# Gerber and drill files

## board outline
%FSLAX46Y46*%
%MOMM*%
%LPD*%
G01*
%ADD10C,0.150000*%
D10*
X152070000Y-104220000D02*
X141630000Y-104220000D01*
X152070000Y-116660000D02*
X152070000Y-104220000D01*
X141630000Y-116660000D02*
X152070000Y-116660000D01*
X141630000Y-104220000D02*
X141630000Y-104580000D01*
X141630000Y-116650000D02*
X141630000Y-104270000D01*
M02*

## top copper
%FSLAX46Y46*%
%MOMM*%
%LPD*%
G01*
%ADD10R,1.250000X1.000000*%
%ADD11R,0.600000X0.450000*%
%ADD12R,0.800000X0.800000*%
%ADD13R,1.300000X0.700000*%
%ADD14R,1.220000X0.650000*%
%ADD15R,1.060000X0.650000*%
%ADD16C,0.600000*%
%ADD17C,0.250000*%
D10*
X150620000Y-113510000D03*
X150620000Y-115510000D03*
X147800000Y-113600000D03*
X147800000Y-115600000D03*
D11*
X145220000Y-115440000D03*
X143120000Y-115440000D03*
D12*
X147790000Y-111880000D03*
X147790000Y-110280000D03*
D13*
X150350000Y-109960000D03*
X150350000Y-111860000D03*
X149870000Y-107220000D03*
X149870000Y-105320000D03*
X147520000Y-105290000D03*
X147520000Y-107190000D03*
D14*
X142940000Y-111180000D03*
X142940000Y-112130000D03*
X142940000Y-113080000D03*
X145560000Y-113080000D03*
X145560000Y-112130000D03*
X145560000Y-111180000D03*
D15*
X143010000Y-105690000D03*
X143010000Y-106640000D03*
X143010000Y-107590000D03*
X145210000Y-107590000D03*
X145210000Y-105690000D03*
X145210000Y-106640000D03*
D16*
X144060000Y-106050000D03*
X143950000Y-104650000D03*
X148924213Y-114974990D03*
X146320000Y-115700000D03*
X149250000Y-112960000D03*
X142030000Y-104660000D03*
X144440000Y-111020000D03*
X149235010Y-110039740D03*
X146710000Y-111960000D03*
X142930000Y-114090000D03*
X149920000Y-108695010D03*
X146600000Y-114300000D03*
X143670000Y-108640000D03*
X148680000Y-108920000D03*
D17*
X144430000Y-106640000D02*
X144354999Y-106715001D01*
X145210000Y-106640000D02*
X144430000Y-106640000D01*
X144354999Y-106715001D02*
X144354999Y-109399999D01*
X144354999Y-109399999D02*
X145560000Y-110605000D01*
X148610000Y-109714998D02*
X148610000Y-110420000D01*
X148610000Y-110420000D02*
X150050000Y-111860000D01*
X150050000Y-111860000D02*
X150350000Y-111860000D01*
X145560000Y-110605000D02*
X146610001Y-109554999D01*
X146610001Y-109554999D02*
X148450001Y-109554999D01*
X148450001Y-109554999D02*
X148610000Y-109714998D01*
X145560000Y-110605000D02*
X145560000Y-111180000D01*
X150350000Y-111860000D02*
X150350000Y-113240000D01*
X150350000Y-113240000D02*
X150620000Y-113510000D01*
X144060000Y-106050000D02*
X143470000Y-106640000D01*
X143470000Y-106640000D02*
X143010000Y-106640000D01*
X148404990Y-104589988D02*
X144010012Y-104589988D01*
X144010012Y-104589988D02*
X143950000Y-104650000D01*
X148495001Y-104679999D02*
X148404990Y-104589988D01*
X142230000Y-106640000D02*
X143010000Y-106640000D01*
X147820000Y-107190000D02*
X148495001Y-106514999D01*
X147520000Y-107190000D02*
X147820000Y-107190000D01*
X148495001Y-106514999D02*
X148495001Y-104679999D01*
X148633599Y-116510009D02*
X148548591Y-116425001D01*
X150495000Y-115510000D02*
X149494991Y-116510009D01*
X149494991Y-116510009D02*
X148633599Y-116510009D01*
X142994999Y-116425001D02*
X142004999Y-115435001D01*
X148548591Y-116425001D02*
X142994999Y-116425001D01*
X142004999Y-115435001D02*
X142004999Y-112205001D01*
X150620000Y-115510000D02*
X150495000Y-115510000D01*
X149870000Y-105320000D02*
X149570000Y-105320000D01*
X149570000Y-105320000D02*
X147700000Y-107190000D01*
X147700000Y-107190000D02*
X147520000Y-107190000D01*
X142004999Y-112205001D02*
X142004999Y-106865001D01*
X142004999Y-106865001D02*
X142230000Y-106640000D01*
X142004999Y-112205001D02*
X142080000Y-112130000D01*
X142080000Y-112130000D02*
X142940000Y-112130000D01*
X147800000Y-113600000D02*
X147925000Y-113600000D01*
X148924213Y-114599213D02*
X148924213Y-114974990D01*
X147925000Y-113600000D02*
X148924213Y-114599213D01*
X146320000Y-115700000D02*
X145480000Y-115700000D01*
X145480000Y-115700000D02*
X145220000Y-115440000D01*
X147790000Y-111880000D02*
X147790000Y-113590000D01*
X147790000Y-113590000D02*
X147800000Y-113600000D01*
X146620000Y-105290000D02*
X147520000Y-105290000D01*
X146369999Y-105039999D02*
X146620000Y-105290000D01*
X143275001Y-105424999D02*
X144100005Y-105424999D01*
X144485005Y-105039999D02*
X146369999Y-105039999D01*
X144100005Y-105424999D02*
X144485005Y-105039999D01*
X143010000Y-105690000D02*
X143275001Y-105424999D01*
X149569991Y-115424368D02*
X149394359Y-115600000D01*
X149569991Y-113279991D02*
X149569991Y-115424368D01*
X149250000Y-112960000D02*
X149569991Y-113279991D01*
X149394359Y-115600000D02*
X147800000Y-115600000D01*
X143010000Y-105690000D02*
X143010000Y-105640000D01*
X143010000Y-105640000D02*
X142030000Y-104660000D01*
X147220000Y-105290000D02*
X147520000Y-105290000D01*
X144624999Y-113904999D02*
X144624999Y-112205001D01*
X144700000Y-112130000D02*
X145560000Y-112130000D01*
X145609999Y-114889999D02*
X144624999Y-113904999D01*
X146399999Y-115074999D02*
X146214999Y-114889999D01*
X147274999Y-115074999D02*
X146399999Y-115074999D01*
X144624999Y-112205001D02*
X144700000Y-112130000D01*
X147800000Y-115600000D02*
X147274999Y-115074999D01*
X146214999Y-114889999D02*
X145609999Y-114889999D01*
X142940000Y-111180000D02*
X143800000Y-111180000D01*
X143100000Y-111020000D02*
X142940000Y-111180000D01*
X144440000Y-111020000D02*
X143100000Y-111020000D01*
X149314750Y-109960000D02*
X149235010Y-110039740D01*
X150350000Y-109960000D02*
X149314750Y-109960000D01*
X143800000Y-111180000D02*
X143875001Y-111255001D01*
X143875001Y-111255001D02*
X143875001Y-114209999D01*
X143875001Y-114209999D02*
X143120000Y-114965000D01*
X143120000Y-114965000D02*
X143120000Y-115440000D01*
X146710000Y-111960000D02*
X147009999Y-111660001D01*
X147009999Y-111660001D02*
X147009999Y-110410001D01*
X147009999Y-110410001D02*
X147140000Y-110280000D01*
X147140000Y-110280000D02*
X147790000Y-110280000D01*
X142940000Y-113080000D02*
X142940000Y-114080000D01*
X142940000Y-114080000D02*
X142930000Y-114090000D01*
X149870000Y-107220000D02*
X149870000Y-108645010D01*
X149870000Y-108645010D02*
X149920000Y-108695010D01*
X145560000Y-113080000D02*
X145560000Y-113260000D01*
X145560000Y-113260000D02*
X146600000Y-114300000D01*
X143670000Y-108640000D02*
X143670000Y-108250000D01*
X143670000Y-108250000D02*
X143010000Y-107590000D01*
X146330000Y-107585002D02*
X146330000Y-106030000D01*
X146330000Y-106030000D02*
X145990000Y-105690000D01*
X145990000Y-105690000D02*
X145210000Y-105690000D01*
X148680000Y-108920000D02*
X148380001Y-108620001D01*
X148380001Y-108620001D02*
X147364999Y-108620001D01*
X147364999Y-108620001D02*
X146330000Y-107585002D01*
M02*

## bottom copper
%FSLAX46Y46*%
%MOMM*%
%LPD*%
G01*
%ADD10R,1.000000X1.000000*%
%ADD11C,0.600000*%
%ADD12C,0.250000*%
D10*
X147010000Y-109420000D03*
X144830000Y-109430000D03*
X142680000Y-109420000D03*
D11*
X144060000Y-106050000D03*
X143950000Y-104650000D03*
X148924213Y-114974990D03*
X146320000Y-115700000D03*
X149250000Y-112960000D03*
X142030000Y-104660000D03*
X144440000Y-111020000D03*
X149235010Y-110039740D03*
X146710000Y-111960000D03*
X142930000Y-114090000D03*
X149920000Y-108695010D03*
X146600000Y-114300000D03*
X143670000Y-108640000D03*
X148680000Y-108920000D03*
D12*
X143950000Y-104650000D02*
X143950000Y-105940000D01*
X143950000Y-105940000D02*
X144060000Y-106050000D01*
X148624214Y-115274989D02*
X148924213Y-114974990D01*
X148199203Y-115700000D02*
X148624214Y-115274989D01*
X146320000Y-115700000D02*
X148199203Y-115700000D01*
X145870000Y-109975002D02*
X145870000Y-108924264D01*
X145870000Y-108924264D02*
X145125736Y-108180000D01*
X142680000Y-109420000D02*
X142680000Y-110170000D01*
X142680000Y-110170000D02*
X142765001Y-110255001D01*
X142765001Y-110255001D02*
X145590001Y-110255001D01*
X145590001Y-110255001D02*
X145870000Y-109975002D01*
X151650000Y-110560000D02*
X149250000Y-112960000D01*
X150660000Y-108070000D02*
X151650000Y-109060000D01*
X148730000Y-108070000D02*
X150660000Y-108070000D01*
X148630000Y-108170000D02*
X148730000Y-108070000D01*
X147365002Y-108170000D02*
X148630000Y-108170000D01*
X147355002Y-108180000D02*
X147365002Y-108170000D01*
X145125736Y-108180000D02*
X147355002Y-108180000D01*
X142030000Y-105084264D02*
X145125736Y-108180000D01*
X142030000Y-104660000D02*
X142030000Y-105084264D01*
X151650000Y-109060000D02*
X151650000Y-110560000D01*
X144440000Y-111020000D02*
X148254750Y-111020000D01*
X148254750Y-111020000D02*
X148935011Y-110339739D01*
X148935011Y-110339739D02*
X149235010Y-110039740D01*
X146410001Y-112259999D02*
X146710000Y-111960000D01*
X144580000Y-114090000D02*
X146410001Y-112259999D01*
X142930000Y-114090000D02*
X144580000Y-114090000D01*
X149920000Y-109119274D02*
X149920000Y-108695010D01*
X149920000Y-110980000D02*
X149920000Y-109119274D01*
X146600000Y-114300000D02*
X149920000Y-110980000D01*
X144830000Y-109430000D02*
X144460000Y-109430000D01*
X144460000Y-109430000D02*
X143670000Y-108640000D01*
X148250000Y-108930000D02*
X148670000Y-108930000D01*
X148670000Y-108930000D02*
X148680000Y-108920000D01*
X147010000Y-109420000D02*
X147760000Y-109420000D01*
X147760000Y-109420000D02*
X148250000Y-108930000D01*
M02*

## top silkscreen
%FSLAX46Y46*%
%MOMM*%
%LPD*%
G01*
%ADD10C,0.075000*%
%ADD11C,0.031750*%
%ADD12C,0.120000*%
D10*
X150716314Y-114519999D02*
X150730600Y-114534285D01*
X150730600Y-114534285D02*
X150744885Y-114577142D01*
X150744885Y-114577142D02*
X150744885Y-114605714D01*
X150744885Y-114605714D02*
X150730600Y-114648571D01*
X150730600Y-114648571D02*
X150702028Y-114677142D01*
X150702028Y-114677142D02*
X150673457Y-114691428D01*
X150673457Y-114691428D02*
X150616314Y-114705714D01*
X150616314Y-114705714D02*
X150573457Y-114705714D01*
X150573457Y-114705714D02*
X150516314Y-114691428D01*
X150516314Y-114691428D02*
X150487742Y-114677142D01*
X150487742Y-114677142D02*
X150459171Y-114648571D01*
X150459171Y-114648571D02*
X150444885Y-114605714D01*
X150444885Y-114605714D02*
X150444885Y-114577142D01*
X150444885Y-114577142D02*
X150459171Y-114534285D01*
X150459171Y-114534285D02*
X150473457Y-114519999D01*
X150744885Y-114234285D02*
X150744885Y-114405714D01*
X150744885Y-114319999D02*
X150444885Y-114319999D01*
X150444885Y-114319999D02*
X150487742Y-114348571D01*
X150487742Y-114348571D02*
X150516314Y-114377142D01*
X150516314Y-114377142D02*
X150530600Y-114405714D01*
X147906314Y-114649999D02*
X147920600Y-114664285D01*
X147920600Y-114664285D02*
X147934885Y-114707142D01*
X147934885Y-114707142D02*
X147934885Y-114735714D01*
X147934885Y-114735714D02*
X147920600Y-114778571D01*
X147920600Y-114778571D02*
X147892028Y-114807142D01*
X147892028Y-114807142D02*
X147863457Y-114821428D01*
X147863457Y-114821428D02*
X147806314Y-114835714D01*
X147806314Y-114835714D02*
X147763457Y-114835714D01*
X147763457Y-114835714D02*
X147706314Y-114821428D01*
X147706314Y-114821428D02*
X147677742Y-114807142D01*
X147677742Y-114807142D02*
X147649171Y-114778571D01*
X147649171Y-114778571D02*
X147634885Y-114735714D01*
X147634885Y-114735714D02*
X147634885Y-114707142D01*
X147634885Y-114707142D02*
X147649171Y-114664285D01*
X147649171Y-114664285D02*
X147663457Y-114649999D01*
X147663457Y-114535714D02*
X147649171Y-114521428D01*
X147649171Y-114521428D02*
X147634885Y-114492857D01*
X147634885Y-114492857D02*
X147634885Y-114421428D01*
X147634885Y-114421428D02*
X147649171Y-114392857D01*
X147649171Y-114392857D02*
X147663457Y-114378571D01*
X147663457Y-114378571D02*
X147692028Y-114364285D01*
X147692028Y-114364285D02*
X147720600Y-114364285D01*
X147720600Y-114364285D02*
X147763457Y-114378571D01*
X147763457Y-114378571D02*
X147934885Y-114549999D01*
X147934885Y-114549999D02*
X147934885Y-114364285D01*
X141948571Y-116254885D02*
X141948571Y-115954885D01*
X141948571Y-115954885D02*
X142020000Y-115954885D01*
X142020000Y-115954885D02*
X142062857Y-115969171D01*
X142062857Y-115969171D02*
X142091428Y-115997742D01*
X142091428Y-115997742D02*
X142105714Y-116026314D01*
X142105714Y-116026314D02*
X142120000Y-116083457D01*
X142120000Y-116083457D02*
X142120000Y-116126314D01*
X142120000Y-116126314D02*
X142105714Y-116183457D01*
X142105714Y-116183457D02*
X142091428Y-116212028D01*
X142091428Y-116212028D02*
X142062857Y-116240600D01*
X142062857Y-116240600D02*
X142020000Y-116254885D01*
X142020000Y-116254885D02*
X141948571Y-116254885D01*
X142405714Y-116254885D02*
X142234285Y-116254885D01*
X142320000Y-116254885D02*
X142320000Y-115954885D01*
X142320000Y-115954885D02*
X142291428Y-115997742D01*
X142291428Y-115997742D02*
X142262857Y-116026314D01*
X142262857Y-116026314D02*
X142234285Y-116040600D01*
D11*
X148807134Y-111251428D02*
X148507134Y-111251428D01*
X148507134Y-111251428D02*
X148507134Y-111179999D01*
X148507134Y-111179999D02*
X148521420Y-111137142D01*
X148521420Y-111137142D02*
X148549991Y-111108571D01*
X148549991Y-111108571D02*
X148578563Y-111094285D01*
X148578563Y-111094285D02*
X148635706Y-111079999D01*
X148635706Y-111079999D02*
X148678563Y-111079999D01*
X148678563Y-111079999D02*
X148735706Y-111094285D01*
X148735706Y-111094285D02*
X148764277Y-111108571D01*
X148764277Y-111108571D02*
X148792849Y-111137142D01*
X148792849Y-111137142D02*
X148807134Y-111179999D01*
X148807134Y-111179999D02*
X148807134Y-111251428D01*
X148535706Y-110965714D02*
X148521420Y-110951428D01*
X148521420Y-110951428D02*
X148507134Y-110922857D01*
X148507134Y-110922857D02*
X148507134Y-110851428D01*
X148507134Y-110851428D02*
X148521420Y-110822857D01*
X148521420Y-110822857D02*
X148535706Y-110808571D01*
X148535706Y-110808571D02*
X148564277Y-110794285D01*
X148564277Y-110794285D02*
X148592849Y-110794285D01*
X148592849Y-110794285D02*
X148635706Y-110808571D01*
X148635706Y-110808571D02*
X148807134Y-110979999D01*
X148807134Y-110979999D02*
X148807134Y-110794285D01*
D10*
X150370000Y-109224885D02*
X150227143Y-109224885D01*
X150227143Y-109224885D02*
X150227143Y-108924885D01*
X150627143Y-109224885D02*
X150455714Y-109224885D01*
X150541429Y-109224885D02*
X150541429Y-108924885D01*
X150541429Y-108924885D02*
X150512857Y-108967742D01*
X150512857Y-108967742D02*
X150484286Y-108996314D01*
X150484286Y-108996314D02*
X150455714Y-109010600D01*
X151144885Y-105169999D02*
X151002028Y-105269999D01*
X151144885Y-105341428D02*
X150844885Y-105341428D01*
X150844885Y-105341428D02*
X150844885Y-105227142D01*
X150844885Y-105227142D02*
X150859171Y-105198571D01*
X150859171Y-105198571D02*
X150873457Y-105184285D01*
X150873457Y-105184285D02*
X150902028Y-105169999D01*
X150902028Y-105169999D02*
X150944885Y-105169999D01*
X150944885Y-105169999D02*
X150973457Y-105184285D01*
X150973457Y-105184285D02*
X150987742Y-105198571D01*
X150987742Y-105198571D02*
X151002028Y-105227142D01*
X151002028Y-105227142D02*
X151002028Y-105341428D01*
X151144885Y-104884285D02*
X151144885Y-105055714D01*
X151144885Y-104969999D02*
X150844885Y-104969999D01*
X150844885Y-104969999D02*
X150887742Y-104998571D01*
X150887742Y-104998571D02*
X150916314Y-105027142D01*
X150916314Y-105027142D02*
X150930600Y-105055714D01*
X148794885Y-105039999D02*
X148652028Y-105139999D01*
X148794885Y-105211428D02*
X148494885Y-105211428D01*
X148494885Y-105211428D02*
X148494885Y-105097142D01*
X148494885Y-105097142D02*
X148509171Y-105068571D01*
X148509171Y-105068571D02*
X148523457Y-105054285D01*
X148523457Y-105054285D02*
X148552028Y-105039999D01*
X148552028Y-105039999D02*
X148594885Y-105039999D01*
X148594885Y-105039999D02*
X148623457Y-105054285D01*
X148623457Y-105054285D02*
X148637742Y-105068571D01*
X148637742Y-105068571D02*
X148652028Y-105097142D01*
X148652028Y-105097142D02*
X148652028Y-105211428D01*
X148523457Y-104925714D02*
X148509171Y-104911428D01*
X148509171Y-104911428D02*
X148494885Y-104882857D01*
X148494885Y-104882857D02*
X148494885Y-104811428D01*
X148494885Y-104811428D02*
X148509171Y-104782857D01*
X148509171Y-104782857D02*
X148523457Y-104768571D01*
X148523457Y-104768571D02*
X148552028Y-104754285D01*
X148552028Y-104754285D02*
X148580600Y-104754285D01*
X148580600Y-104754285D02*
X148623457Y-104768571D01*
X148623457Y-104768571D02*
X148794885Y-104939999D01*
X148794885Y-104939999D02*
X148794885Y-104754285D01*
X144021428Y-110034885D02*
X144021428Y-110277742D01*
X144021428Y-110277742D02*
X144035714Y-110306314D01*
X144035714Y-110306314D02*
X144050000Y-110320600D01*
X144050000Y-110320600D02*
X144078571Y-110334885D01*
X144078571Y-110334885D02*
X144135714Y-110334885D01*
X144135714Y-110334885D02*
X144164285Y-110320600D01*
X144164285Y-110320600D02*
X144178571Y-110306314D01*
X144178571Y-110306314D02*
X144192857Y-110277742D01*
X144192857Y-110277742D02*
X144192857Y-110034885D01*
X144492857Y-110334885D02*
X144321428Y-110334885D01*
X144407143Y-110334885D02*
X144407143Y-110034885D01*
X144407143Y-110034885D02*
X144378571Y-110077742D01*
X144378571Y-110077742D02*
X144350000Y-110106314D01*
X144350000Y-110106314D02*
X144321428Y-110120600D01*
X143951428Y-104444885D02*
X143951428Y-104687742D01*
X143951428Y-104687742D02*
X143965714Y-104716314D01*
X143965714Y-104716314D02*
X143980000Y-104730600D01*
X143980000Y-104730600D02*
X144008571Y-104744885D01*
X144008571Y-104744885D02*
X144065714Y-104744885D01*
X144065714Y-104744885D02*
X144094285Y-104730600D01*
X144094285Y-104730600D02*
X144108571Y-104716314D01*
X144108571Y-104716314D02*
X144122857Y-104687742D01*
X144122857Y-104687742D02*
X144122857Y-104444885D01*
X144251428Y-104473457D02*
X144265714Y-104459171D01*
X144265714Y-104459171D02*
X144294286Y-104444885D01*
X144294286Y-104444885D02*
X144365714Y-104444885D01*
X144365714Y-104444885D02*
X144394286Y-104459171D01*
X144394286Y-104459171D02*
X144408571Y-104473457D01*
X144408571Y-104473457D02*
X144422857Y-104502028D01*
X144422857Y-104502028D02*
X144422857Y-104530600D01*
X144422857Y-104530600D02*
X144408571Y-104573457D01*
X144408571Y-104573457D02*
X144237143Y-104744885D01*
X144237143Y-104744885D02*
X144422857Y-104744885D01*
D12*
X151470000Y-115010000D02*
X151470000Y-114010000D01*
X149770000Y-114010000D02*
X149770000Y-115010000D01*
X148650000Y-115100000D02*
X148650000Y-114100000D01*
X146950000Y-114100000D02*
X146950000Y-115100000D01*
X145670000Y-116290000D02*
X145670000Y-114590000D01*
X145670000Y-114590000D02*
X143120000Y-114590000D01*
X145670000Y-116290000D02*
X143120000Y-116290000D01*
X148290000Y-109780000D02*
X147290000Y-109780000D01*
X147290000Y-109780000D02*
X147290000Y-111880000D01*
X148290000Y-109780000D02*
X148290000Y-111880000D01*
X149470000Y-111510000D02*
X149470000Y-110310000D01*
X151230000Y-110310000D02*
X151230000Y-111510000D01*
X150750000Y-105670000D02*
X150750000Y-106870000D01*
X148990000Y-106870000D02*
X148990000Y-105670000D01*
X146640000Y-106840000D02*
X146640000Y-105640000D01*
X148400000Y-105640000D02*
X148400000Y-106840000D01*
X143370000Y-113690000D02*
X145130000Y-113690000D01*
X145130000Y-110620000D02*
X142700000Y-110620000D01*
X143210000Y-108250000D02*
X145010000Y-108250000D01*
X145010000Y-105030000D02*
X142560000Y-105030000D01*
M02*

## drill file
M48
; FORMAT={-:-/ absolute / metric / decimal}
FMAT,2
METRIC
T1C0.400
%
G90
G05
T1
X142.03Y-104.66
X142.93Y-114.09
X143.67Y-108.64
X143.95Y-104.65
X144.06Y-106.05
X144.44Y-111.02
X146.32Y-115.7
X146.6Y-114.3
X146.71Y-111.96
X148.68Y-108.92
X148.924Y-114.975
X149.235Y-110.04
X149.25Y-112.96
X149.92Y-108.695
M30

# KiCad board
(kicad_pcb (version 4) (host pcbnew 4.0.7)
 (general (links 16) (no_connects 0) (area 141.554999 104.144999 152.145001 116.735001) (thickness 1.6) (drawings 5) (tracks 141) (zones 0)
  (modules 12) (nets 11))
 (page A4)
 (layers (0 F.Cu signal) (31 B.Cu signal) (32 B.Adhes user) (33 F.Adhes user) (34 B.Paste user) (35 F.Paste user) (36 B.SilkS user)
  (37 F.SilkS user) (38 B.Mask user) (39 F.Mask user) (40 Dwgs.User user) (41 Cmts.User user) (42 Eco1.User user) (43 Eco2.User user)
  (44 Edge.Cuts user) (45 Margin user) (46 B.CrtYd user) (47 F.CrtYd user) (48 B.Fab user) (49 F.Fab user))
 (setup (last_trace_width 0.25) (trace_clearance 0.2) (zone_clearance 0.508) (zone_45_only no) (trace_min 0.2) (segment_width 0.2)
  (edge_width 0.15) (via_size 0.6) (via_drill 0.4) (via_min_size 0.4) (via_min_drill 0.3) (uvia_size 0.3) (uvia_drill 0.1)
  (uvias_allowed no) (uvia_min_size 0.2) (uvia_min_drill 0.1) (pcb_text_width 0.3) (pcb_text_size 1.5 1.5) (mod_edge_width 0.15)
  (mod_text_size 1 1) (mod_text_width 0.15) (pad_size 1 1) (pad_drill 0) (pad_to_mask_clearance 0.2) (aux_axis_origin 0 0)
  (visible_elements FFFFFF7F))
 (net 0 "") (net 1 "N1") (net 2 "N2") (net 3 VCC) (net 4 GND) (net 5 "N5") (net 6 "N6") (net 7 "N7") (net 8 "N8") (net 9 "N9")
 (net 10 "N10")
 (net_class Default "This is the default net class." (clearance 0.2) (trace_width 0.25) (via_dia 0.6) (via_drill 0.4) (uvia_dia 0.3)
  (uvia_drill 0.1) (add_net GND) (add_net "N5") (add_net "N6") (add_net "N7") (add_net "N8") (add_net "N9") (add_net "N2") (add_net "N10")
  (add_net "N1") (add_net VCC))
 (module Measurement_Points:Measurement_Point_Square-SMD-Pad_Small (layer B.Cu) (at 147.01 109.42)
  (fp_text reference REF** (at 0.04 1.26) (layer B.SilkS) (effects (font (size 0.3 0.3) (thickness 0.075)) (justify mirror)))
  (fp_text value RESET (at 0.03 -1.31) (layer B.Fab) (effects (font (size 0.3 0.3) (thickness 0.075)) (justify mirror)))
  (pad 1 smd rect (at 0 0) (size 1 1) (layers B.Cu B.Mask) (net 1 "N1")))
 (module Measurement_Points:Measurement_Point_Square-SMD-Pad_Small (layer B.Cu) (at 144.83 109.43)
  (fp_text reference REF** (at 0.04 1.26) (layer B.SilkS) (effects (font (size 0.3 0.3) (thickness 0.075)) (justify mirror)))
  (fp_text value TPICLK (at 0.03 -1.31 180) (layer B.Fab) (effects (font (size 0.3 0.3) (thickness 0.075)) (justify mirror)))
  (pad 1 smd rect (at 0 0) (size 1 1) (layers B.Cu B.Mask) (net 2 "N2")))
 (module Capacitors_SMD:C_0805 (layer F.Cu) (at 150.62 114.51 270)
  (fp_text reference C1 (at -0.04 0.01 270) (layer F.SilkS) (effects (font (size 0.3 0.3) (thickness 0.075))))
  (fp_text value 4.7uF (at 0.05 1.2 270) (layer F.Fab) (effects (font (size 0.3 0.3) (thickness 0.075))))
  (fp_line (start 0.5 -0.85) (end -0.5 -0.85) (layer F.SilkS) (width 0.12))
  (fp_line (start -0.5 0.85) (end 0.5 0.85) (layer F.SilkS) (width 0.12))
  (pad 1 smd rect (at -1 0 270) (size 1 1.25) (layers F.Cu F.Paste F.Mask) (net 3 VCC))
  (pad 2 smd rect (at 1 0 270) (size 1 1.25) (layers F.Cu F.Paste F.Mask) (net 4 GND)))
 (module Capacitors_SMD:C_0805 (layer F.Cu) (at 147.8 114.6 270)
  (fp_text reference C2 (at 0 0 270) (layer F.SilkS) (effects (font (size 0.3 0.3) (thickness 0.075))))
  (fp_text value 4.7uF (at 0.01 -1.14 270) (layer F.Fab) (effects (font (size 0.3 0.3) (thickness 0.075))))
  (fp_line (start 0.5 -0.85) (end -0.5 -0.85) (layer F.SilkS) (width 0.12))
  (fp_line (start -0.5 0.85) (end 0.5 0.85) (layer F.SilkS) (width 0.12))
  (pad 1 smd rect (at -1 0 270) (size 1 1.25) (layers F.Cu F.Paste F.Mask) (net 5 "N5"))
  (pad 2 smd rect (at 1 0 270) (size 1 1.25) (layers F.Cu F.Paste F.Mask) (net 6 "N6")))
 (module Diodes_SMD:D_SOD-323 (layer F.Cu) (at 144.17 115.44 180)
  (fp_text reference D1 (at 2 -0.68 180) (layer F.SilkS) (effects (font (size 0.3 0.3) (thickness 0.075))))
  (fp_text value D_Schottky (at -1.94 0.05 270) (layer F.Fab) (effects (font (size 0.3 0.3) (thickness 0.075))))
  (fp_line (start -1.5 -0.85) (end -1.5 0.85) (layer F.SilkS) (width 0.12))
  (fp_line (start -1.5 0.85) (end 1.05 0.85) (layer F.SilkS) (width 0.12))
  (fp_line (start -1.5 -0.85) (end 1.05 -0.85) (layer F.SilkS) (width 0.12))
  (pad 1 smd rect (at -1.05 0 180) (size 0.6 0.45) (layers F.Cu F.Paste F.Mask) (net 5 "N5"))
  (pad 2 smd rect (at 1.05 0 180) (size 0.6 0.45) (layers F.Cu F.Paste F.Mask) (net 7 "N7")))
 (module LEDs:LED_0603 (layer F.Cu) (at 147.79 111.08 270)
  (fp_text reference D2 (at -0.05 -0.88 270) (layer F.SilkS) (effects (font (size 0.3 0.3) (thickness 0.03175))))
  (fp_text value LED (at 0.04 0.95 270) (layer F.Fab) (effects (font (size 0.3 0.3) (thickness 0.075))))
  (fp_line (start -1.3 -0.5) (end -1.3 0.5) (layer F.SilkS) (width 0.12))
  (fp_line (start -1.3 0.5) (end 0.8 0.5) (layer F.SilkS) (width 0.12))
  (fp_line (start -1.3 -0.5) (end 0.8 -0.5) (layer F.SilkS) (width 0.12))
  (pad 2 smd rect (at 0.8 0 90) (size 0.8 0.8) (layers F.Cu F.Paste F.Mask) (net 5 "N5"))
  (pad 1 smd rect (at -0.8 0 90) (size 0.8 0.8) (layers F.Cu F.Paste F.Mask) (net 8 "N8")))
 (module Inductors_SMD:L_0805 (layer F.Cu) (at 150.35 110.91 270)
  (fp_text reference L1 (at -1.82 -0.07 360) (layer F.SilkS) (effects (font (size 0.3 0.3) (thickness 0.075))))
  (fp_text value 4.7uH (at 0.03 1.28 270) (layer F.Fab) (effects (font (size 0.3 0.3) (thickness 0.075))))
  (fp_line (start 0.6 0.88) (end -0.6 0.88) (layer F.SilkS) (width 0.12))
  (fp_line (start -0.6 -0.88) (end 0.6 -0.88) (layer F.SilkS) (width 0.12))
  (pad 1 smd rect (at -0.95 0 270) (size 0.7 1.3) (layers F.Cu F.Paste F.Mask) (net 7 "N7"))
  (pad 2 smd rect (at 0.95 0 270) (size 0.7 1.3) (layers F.Cu F.Paste F.Mask) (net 3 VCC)))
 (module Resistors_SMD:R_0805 (layer F.Cu) (at 149.87 106.27 90)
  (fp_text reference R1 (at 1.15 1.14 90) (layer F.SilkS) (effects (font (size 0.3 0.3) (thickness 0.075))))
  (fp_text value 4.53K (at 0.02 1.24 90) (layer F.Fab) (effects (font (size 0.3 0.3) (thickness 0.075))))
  (fp_line (start 0.6 0.88) (end -0.6 0.88) (layer F.SilkS) (width 0.12))
  (fp_line (start -0.6 -0.88) (end 0.6 -0.88) (layer F.SilkS) (width 0.12))
  (pad 1 smd rect (at -0.95 0 90) (size 0.7 1.3) (layers F.Cu F.Paste F.Mask) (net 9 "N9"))
  (pad 2 smd rect (at 0.95 0 90) (size 0.7 1.3) (layers F.Cu F.Paste F.Mask) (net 4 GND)))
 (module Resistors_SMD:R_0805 (layer F.Cu) (at 147.52 106.24 270)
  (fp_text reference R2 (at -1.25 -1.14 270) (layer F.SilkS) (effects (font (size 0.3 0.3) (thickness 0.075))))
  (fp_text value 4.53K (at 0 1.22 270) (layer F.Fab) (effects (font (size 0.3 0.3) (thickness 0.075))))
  (fp_line (start 0.6 0.88) (end -0.6 0.88) (layer F.SilkS) (width 0.12))
  (fp_line (start -0.6 -0.88) (end 0.6 -0.88) (layer F.SilkS) (width 0.12))
  (pad 1 smd rect (at -0.95 0 270) (size 0.7 1.3) (layers F.Cu F.Paste F.Mask) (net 6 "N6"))
  (pad 2 smd rect (at 0.95 0 270) (size 0.7 1.3) (layers F.Cu F.Paste F.Mask) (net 4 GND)))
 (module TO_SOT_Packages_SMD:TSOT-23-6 (layer F.Cu) (at 144.25 112.13)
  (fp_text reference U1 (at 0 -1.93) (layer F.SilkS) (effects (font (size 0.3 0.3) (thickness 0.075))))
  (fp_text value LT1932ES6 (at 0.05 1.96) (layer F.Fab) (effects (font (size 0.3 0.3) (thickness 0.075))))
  (fp_line (start -0.88 1.56) (end 0.88 1.56) (layer F.SilkS) (width 0.12))
  (fp_line (start 0.88 -1.51) (end -1.55 -1.51) (layer F.SilkS) (width 0.12))
  (pad 1 smd rect (at -1.31 -0.95) (size 1.22 0.65) (layers F.Cu F.Paste F.Mask) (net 7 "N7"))
  (pad 2 smd rect (at -1.31 0) (size 1.22 0.65) (layers F.Cu F.Paste F.Mask) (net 4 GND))
  (pad 3 smd rect (at -1.31 0.95) (size 1.22 0.65) (layers F.Cu F.Paste F.Mask) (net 8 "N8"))
  (pad 4 smd rect (at 1.31 0.95) (size 1.22 0.65) (layers F.Cu F.Paste F.Mask) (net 9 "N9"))
  (pad 5 smd rect (at 1.31 0) (size 1.22 0.65) (layers F.Cu F.Paste F.Mask) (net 6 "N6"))
  (pad 6 smd rect (at 1.31 -0.95) (size 1.22 0.65) (layers F.Cu F.Paste F.Mask) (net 3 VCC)))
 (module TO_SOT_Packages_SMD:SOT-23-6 (layer F.Cu) (at 144.11 106.64)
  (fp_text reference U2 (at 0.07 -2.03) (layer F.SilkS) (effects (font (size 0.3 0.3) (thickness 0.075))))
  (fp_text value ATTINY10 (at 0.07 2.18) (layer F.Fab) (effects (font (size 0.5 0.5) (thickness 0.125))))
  (fp_line (start -0.9 1.61) (end 0.9 1.61) (layer F.SilkS) (width 0.12))
  (fp_line (start 0.9 -1.61) (end -1.55 -1.61) (layer F.SilkS) (width 0.12))
  (pad 1 smd rect (at -1.1 -0.95) (size 1.06 0.65) (layers F.Cu F.Paste F.Mask) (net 6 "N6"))
  (pad 2 smd rect (at -1.1 0) (size 1.06 0.65) (layers F.Cu F.Paste F.Mask) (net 4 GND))
  (pad 3 smd rect (at -1.1 0.95) (size 1.06 0.65) (layers F.Cu F.Paste F.Mask) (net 2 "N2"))
  (pad 4 smd rect (at 1.1 0.95) (size 1.06 0.65) (layers F.Cu F.Paste F.Mask) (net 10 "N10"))
  (pad 6 smd rect (at 1.1 -0.95) (size 1.06 0.65) (layers F.Cu F.Paste F.Mask) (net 1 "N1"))
  (pad 5 smd rect (at 1.1 0) (size 1.06 0.65) (layers F.Cu F.Paste F.Mask) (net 3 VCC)))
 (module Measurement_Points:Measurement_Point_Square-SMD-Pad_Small (layer B.Cu) (at 142.68 109.42)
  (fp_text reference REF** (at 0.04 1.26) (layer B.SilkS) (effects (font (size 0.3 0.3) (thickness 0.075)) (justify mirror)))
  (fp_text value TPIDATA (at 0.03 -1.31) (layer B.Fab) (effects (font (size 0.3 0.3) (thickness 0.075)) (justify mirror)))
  (pad 1 smd rect (at 0 0) (size 1 1) (layers B.Cu B.Mask) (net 6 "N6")))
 (gr_line (start 152.07 104.22) (end 141.63 104.22) (angle 90) (layer Edge.Cuts) (width 0.15))
 (gr_line (start 152.07 116.66) (end 152.07 104.22) (angle 90) (layer Edge.Cuts) (width 0.15))
 (gr_line (start 141.63 116.66) (end 152.07 116.66) (angle 90) (layer Edge.Cuts) (width 0.15))
 (gr_line (start 141.63 104.22) (end 141.63 104.58) (angle 90) (layer Edge.Cuts) (width 0.15))
 (gr_line (start 141.63 116.65) (end 141.63 104.27) (angle 90) (layer Edge.Cuts) (width 0.15))
 (segment (start 144.43 106.64) (end 144.354999 106.715001) (width 0.25) (layer F.Cu) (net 3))
 (segment (start 145.21 106.64) (end 144.43 106.64) (width 0.25) (layer F.Cu) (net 3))
 (segment (start 144.354999 106.715001) (end 144.354999 109.399999) (width 0.25) (layer F.Cu) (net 3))
 (segment (start 144.354999 109.399999) (end 145.56 110.605) (width 0.25) (layer F.Cu) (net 3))
 (segment (start 148.61 109.714998) (end 148.61 110.42) (width 0.25) (layer F.Cu) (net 3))
 (segment (start 148.61 110.42) (end 150.05 111.86) (width 0.25) (layer F.Cu) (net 3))
 (segment (start 150.05 111.86) (end 150.35 111.86) (width 0.25) (layer F.Cu) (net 3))
 (segment (start 145.56 110.605) (end 146.610001 109.554999) (width 0.25) (layer F.Cu) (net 3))
 (segment (start 146.610001 109.554999) (end 148.450001 109.554999) (width 0.25) (layer F.Cu) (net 3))
 (segment (start 148.450001 109.554999) (end 148.61 109.714998) (width 0.25) (layer F.Cu) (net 3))
 (segment (start 145.56 110.605) (end 145.56 111.18) (width 0.25) (layer F.Cu) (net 3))
 (segment (start 150.35 111.86) (end 150.35 113.24) (width 0.25) (layer F.Cu) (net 3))
 (segment (start 150.35 113.24) (end 150.62 113.51) (width 0.25) (layer F.Cu) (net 3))
 (segment (start 144.06 106.05) (end 143.47 106.64) (width 0.25) (layer F.Cu) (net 4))
 (segment (start 143.47 106.64) (end 143.01 106.64) (width 0.25) (layer F.Cu) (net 4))
 (segment (start 143.95 104.65) (end 143.95 105.94) (width 0.25) (layer B.Cu) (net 4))
 (segment (start 143.95 105.94) (end 144.06 106.05) (width 0.25) (layer B.Cu) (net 4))
 (via (at 144.06 106.05) (size 0.6) (drill 0.4) (layers F.Cu B.Cu) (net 4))
 (segment (start 148.40499 104.589988) (end 144.010012 104.589988) (width 0.25) (layer F.Cu) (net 4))
 (segment (start 144.010012 104.589988) (end 143.95 104.65) (width 0.25) (layer F.Cu) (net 4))
 (segment (start 148.495001 104.679999) (end 148.40499 104.589988) (width 0.25) (layer F.Cu) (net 4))
 (via (at 143.95 104.65) (size 0.6) (drill 0.4) (layers F.Cu B.Cu) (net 4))
 (segment (start 142.23 106.64) (end 143.01 106.64) (width 0.25) (layer F.Cu) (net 4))
 (segment (start 147.82 107.19) (end 148.495001 106.514999) (width 0.25) (layer F.Cu) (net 4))
 (segment (start 147.52 107.19) (end 147.82 107.19) (width 0.25) (layer F.Cu) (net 4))
 (segment (start 148.495001 106.514999) (end 148.495001 104.679999) (width 0.25) (layer F.Cu) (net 4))
 (segment (start 148.633599 116.510009) (end 148.548591 116.425001) (width 0.25) (layer F.Cu) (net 4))
 (segment (start 150.495 115.51) (end 149.494991 116.510009) (width 0.25) (layer F.Cu) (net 4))
 (segment (start 149.494991 116.510009) (end 148.633599 116.510009) (width 0.25) (layer F.Cu) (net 4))
 (segment (start 142.994999 116.425001) (end 142.004999 115.435001) (width 0.25) (layer F.Cu) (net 4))
 (segment (start 148.548591 116.425001) (end 142.994999 116.425001) (width 0.25) (layer F.Cu) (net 4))
 (segment (start 142.004999 115.435001) (end 142.004999 112.205001) (width 0.25) (layer F.Cu) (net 4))
 (segment (start 150.62 115.51) (end 150.495 115.51) (width 0.25) (layer F.Cu) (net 4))
 (segment (start 149.87 105.32) (end 149.57 105.32) (width 0.25) (layer F.Cu) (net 4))
 (segment (start 149.57 105.32) (end 147.7 107.19) (width 0.25) (layer F.Cu) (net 4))
 (segment (start 147.7 107.19) (end 147.52 107.19) (width 0.25) (layer F.Cu) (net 4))
 (segment (start 142.004999 112.205001) (end 142.004999 106.865001) (width 0.25) (layer F.Cu) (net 4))
 (segment (start 142.004999 106.865001) (end 142.23 106.64) (width 0.25) (layer F.Cu) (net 4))
 (segment (start 142.004999 112.205001) (end 142.08 112.13) (width 0.25) (layer F.Cu) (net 4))
 (segment (start 142.08 112.13) (end 142.94 112.13) (width 0.25) (layer F.Cu) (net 4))
 (segment (start 148.624214 115.274989) (end 148.924213 114.97499) (width 0.25) (layer B.Cu) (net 5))
 (segment (start 148.199203 115.7) (end 148.624214 115.274989) (width 0.25) (layer B.Cu) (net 5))
 (segment (start 147.8 113.6) (end 147.925 113.6) (width 0.25) (layer F.Cu) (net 5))
 (segment (start 146.32 115.7) (end 148.199203 115.7) (width 0.25) (layer B.Cu) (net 5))
 (segment (start 148.924213 114.599213) (end 148.924213 114.97499) (width 0.25) (layer F.Cu) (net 5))
 (segment (start 147.925 113.6) (end 148.924213 114.599213) (width 0.25) (layer F.Cu) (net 5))
 (via (at 148.924213 114.97499) (size 0.6) (drill 0.4) (layers F.Cu B.Cu) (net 5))
 (segment (start 146.32 115.7) (end 145.48 115.7) (width 0.25) (layer F.Cu) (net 5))
 (segment (start 145.48 115.7) (end 145.22 115.44) (width 0.25) (layer F.Cu) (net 5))
 (via (at 146.32 115.7) (size 0.6) (drill 0.4) (layers F.Cu B.Cu) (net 5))
 (segment (start 147.79 111.88) (end 147.79 113.59) (width 0.25) (layer F.Cu) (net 5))
 (segment (start 147.79 113.59) (end 147.8 113.6) (width 0.25) (layer F.Cu) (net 5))
 (segment (start 145.87 109.975002) (end 145.87 108.924264) (width 0.25) (layer B.Cu) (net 6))
 (segment (start 145.87 108.924264) (end 145.125736 108.18) (width 0.25) (layer B.Cu) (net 6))
 (segment (start 142.68 109.42) (end 142.68 110.17) (width 0.25) (layer B.Cu) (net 6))
 (segment (start 142.68 110.17) (end 142.765001 110.255001) (width 0.25) (layer B.Cu) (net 6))
 (segment (start 142.765001 110.255001) (end 145.590001 110.255001) (width 0.25) (layer B.Cu) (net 6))
 (segment (start 145.590001 110.255001) (end 145.87 109.975002) (width 0.25) (layer B.Cu) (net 6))
 (segment (start 146.62 105.29) (end 147.52 105.29) (width 0.25) (layer F.Cu) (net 6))
 (segment (start 146.369999 105.039999) (end 146.62 105.29) (width 0.25) (layer F.Cu) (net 6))
 (segment (start 143.275001 105.424999) (end 144.100005 105.424999) (width 0.25) (layer F.Cu) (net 6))
 (segment (start 144.485005 105.039999) (end 146.369999 105.039999) (width 0.25) (layer F.Cu) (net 6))
 (segment (start 144.100005 105.424999) (end 144.485005 105.039999) (width 0.25) (layer F.Cu) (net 6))
 (segment (start 143.01 105.69) (end 143.275001 105.424999) (width 0.25) (layer F.Cu) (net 6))
 (segment (start 151.65 110.56) (end 149.25 112.96) (width 0.25) (layer B.Cu) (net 6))
 (segment (start 150.66 108.07) (end 151.65 109.06) (width 0.25) (layer B.Cu) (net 6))
 (segment (start 148.73 108.07) (end 150.66 108.07) (width 0.25) (layer B.Cu) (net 6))
 (segment (start 148.63 108.17) (end 148.73 108.07) (width 0.25) (layer B.Cu) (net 6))
 (segment (start 147.365002 108.17) (end 148.63 108.17) (width 0.25) (layer B.Cu) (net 6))
 (segment (start 147.355002 108.18) (end 147.365002 108.17) (width 0.25) (layer B.Cu) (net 6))
 (segment (start 145.125736 108.18) (end 147.355002 108.18) (width 0.25) (layer B.Cu) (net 6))
 (segment (start 142.03 105.084264) (end 145.125736 108.18) (width 0.25) (layer B.Cu) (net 6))
 (segment (start 142.03 104.66) (end 142.03 105.084264) (width 0.25) (layer B.Cu) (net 6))
 (segment (start 151.65 109.06) (end 151.65 110.56) (width 0.25) (layer B.Cu) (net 6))
 (segment (start 149.569991 115.424368) (end 149.394359 115.6) (width 0.25) (layer F.Cu) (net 6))
 (segment (start 149.569991 113.279991) (end 149.569991 115.424368) (width 0.25) (layer F.Cu) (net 6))
 (segment (start 149.25 112.96) (end 149.569991 113.279991) (width 0.25) (layer F.Cu) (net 6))
 (segment (start 149.394359 115.6) (end 147.8 115.6) (width 0.25) (layer F.Cu) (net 6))
 (via (at 149.25 112.96) (size 0.6) (drill 0.4) (layers F.Cu B.Cu) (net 6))
 (segment (start 143.01 105.69) (end 143.01 105.64) (width 0.25) (layer F.Cu) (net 6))
 (via (at 142.03 104.66) (size 0.6) (drill 0.4) (layers F.Cu B.Cu) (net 6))
 (segment (start 143.01 105.64) (end 142.03 104.66) (width 0.25) (layer F.Cu) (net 6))
 (segment (start 147.22 105.29) (end 147.52 105.29) (width 0.25) (layer F.Cu) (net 6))
 (segment (start 144.624999 113.904999) (end 144.624999 112.205001) (width 0.25) (layer F.Cu) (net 6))
 (segment (start 144.7 112.13) (end 145.56 112.13) (width 0.25) (layer F.Cu) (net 6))
 (segment (start 145.609999 114.889999) (end 144.624999 113.904999) (width 0.25) (layer F.Cu) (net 6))
 (segment (start 146.399999 115.074999) (end 146.214999 114.889999) (width 0.25) (layer F.Cu) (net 6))
 (segment (start 147.274999 115.074999) (end 146.399999 115.074999) (width 0.25) (layer F.Cu) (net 6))
 (segment (start 144.624999 112.205001) (end 144.7 112.13) (width 0.25) (layer F.Cu) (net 6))
 (segment (start 147.8 115.6) (end 147.274999 115.074999) (width 0.25) (layer F.Cu) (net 6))
 (segment (start 146.214999 114.889999) (end 145.609999 114.889999) (width 0.25) (layer F.Cu) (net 6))
 (segment (start 142.94 111.18) (end 143.8 111.18) (width 0.25) (layer F.Cu) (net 7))
 (segment (start 144.44 111.02) (end 148.25475 111.02) (width 0.25) (layer B.Cu) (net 7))
 (segment (start 148.25475 111.02) (end 148.935011 110.339739) (width 0.25) (layer B.Cu) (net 7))
 (segment (start 143.1 111.02) (end 142.94 111.18) (width 0.25) (layer F.Cu) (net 7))
 (segment (start 144.44 111.02) (end 143.1 111.02) (width 0.25) (layer F.Cu) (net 7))
 (via (at 144.44 111.02) (size 0.6) (drill 0.4) (layers F.Cu B.Cu) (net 7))
 (segment (start 148.935011 110.339739) (end 149.23501 110.03974) (width 0.25) (layer B.Cu) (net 7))
 (segment (start 149.31475 109.96) (end 149.23501 110.03974) (width 0.25) (layer F.Cu) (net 7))
 (segment (start 150.35 109.96) (end 149.31475 109.96) (width 0.25) (layer F.Cu) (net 7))
 (via (at 149.23501 110.03974) (size 0.6) (drill 0.4) (layers F.Cu B.Cu) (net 7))
 (segment (start 143.8 111.18) (end 143.875001 111.255001) (width 0.25) (layer F.Cu) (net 7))
 (segment (start 143.875001 111.255001) (end 143.875001 114.209999) (width 0.25) (layer F.Cu) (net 7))
 (segment (start 143.875001 114.209999) (end 143.12 114.965) (width 0.25) (layer F.Cu) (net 7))
 (segment (start 143.12 114.965) (end 143.12 115.44) (width 0.25) (layer F.Cu) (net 7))
 (segment (start 146.410001 112.259999) (end 146.71 111.96) (width 0.25) (layer B.Cu) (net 8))
 (segment (start 144.58 114.09) (end 146.410001 112.259999) (width 0.25) (layer B.Cu) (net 8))
 (segment (start 142.93 114.09) (end 144.58 114.09) (width 0.25) (layer B.Cu) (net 8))
 (segment (start 146.71 111.96) (end 147.009999 111.660001) (width 0.25) (layer F.Cu) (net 8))
 (segment (start 147.009999 111.660001) (end 147.009999 110.410001) (width 0.25) (layer F.Cu) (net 8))
 (segment (start 147.009999 110.410001) (end 147.14 110.28) (width 0.25) (layer F.Cu) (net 8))
 (segment (start 147.14 110.28) (end 147.79 110.28) (width 0.25) (layer F.Cu) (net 8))
 (via (at 146.71 111.96) (size 0.6) (drill 0.4) (layers F.Cu B.Cu) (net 8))
 (segment (start 142.94 113.08) (end 142.94 114.08) (width 0.25) (layer F.Cu) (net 8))
 (segment (start 142.94 114.08) (end 142.93 114.09) (width 0.25) (layer F.Cu) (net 8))
 (via (at 142.93 114.09) (size 0.6) (drill 0.4) (layers F.Cu B.Cu) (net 8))
 (segment (start 149.87 107.22) (end 149.87 108.64501) (width 0.25) (layer F.Cu) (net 9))
 (segment (start 149.92 109.119274) (end 149.92 108.69501) (width 0.25) (layer B.Cu) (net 9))
 (segment (start 149.92 110.98) (end 149.92 109.119274) (width 0.25) (layer B.Cu) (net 9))
 (segment (start 149.87 108.64501) (end 149.92 108.69501) (width 0.25) (layer F.Cu) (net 9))
 (segment (start 146.6 114.3) (end 149.92 110.98) (width 0.25) (layer B.Cu) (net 9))
 (via (at 149.92 108.69501) (size 0.6) (drill 0.4) (layers F.Cu B.Cu) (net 9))
 (segment (start 145.56 113.08) (end 145.56 113.26) (width 0.25) (layer F.Cu) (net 9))
 (via (at 146.6 114.3) (size 0.6) (drill 0.4) (layers F.Cu B.Cu) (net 9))
 (segment (start 145.56 113.26) (end 146.6 114.3) (width 0.25) (layer F.Cu) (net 9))
 (segment (start 143.67 108.64) (end 143.67 108.25) (width 0.25) (layer F.Cu) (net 2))
 (segment (start 143.67 108.25) (end 143.01 107.59) (width 0.25) (layer F.Cu) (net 2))
 (segment (start 144.83 109.43) (end 144.46 109.43) (width 0.25) (layer B.Cu) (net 2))
 (segment (start 144.46 109.43) (end 143.67 108.64) (width 0.25) (layer B.Cu) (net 2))
 (via (at 143.67 108.64) (size 0.6) (drill 0.4) (layers F.Cu B.Cu) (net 2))
 (segment (start 146.33 107.585002) (end 146.33 106.03) (width 0.25) (layer F.Cu) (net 1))
 (segment (start 146.33 106.03) (end 145.99 105.69) (width 0.25) (layer F.Cu) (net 1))
 (segment (start 145.99 105.69) (end 145.21 105.69) (width 0.25) (layer F.Cu) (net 1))
 (segment (start 148.68 108.92) (end 148.380001 108.620001) (width 0.25) (layer F.Cu) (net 1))
 (segment (start 148.380001 108.620001) (end 147.364999 108.620001) (width 0.25) (layer F.Cu) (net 1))
 (segment (start 147.364999 108.620001) (end 146.33 107.585002) (width 0.25) (layer F.Cu) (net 1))
 (segment (start 148.25 108.93) (end 148.67 108.93) (width 0.25) (layer B.Cu) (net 1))
 (segment (start 148.67 108.93) (end 148.68 108.92) (width 0.25) (layer B.Cu) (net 1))
 (via (at 148.68 108.92) (size 0.6) (drill 0.4) (layers F.Cu B.Cu) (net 1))
 (segment (start 147.01 109.42) (end 147.76 109.42) (width 0.25) (layer B.Cu) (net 1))
 (segment (start 147.76 109.42) (end 148.25 108.93) (width 0.25) (layer B.Cu) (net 1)))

